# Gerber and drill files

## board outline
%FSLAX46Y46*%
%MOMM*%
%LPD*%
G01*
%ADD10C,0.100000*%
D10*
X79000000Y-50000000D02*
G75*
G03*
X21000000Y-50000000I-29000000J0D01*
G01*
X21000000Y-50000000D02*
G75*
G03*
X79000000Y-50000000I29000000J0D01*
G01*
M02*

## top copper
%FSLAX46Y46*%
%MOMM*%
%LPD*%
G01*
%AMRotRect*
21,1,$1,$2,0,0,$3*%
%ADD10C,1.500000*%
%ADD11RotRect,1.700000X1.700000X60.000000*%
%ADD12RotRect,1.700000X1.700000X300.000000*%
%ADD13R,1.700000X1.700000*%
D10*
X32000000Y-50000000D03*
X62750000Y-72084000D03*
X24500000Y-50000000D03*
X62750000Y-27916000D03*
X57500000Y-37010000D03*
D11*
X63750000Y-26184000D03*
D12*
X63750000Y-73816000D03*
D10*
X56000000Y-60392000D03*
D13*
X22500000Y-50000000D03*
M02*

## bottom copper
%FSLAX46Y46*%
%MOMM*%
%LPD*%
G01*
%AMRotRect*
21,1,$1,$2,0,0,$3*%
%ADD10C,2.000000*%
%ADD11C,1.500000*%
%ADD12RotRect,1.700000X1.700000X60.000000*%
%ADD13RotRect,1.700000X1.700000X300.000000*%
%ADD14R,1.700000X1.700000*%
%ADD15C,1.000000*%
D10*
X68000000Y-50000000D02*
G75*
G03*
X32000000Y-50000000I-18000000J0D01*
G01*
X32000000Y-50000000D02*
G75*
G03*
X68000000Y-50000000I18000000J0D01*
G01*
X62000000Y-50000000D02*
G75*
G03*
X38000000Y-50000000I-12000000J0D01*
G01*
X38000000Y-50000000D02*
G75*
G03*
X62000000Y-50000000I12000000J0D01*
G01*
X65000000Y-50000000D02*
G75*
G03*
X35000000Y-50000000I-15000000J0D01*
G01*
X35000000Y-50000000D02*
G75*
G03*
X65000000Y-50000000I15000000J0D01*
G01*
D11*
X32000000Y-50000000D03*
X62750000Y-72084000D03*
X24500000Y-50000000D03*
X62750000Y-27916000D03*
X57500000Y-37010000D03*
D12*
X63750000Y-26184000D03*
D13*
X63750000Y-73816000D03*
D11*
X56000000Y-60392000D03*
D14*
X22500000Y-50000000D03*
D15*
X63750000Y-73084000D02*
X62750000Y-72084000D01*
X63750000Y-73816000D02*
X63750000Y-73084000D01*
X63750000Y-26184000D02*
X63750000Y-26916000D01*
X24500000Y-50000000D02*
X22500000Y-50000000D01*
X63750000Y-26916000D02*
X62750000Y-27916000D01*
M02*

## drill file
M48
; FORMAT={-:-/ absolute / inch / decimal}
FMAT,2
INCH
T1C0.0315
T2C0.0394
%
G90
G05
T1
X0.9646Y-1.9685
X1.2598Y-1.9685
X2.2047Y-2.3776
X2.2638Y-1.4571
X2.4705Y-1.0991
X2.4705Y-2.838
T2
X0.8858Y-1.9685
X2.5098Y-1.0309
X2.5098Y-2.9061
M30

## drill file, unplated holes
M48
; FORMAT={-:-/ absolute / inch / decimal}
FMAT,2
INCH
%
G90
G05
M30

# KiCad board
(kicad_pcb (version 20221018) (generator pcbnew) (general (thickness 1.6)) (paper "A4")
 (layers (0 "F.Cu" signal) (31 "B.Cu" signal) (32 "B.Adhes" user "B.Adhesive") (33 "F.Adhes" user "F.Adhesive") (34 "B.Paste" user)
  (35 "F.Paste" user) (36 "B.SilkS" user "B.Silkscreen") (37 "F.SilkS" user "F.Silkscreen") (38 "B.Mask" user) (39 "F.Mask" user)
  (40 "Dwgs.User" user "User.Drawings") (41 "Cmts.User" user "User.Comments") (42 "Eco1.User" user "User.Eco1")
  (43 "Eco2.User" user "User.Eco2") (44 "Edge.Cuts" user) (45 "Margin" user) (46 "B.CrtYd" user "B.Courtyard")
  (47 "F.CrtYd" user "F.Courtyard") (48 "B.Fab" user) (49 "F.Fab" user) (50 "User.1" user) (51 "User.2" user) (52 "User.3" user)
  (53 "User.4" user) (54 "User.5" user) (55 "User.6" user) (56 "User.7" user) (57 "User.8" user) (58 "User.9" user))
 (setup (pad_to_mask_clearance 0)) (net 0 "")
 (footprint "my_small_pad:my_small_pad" (layer "F.Cu") (at 32 50)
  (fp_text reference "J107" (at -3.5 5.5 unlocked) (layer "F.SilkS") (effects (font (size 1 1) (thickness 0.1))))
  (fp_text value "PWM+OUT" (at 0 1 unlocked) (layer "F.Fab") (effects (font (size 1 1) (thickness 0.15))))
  (pad "1" thru_hole circle (at 0 0) (size 1.5 1.5) (drill 0.8) (layers "*.Cu" "*.Mask")))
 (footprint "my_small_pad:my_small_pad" (layer "F.Cu") (at 62.75 72.084)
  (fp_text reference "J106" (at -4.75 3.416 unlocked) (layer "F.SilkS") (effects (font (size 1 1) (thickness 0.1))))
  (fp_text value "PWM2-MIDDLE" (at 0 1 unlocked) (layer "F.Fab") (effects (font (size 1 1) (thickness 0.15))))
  (pad "1" thru_hole circle (at 0 0) (size 1.5 1.5) (drill 0.8) (layers "*.Cu" "*.Mask")))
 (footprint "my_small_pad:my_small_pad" (layer "F.Cu") (at 24.5 50)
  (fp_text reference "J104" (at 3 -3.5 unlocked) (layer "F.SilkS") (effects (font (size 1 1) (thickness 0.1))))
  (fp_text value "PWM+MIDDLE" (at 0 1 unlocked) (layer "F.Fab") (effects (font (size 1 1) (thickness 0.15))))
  (pad "1" thru_hole circle (at 0 0) (size 1.5 1.5) (drill 0.8) (layers "*.Cu" "*.Mask")))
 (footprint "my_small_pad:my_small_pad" (layer "F.Cu") (at 62.75 27.916)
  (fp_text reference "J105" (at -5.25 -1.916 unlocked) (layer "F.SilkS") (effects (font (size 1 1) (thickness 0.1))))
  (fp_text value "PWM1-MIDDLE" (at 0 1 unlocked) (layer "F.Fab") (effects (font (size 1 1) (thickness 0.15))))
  (pad "1" thru_hole circle (at 0 0) (size 1.5 1.5) (drill 0.8) (layers "*.Cu" "*.Mask")))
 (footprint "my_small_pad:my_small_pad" (layer "F.Cu") (at 57.5 37.01)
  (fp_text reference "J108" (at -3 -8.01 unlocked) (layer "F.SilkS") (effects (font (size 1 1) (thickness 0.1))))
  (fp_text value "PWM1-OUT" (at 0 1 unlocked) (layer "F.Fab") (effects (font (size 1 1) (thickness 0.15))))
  (pad "1" thru_hole circle (at 0 0) (size 1.5 1.5) (drill 0.8) (layers "*.Cu" "*.Mask")))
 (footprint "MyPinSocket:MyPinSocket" (layer "F.Cu") (at 63.75 26.184 60)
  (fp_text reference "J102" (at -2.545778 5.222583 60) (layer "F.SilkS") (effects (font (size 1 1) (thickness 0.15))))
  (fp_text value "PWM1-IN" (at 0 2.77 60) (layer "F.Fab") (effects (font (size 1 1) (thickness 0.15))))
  (pad "1" thru_hole rect (at 0 0 60) (size 1.7 1.7) (drill 1) (layers "*.Cu" "*.Mask")))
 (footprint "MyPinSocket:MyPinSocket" (layer "F.Cu") (at 63.75 73.816 -60)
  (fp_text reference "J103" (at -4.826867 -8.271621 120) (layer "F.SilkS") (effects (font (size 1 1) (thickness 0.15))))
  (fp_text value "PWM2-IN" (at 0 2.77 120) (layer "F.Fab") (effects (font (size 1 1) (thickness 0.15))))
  (pad "1" thru_hole rect (at 0 0 300) (size 1.7 1.7) (drill 1) (layers "*.Cu" "*.Mask")))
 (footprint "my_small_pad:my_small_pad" (layer "F.Cu") (at 56 60.392)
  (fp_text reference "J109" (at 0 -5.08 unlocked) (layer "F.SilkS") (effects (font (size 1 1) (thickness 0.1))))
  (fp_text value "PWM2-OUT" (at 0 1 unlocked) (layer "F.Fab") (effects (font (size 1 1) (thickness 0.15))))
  (pad "1" thru_hole circle (at 0 0) (size 1.5 1.5) (drill 0.8) (layers "*.Cu" "*.Mask")))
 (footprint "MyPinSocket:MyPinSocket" (layer "F.Cu") (at 22.5 50)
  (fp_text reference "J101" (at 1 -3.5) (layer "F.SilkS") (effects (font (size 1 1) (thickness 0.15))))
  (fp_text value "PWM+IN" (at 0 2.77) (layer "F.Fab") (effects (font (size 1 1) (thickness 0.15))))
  (pad "1" thru_hole rect (at 0 0) (size 1.7 1.7) (drill 1) (layers "*.Cu" "*.Mask")))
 (gr_circle (center 50 50) (end 68 50) (stroke (width 2) (type default)) (fill none) (layer "B.Cu"))
 (gr_circle (center 50 50) (end 62 50) (stroke (width 2) (type default)) (fill none) (layer "B.Cu"))
 (gr_circle (center 50 50) (end 65 50) (stroke (width 2) (type default)) (fill none) (layer "B.Cu"))
 (gr_circle (center 50 50) (end 79 50) (stroke (width 0.1) (type default)) (fill none) (layer "Edge.Cuts"))
 (segment (start 63.75 73.084) (end 62.75 72.084) (width 1) (layer "B.Cu") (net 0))
 (segment (start 63.75 73.816) (end 63.75 73.084) (width 1) (layer "B.Cu") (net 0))
 (segment (start 63.75 26.184) (end 63.75 26.916) (width 1) (layer "B.Cu") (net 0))
 (segment (start 24.5 50) (end 22.5 50) (width 1) (layer "B.Cu") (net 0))
 (segment (start 63.75 26.916) (end 62.75 27.916) (width 1) (layer "B.Cu") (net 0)))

